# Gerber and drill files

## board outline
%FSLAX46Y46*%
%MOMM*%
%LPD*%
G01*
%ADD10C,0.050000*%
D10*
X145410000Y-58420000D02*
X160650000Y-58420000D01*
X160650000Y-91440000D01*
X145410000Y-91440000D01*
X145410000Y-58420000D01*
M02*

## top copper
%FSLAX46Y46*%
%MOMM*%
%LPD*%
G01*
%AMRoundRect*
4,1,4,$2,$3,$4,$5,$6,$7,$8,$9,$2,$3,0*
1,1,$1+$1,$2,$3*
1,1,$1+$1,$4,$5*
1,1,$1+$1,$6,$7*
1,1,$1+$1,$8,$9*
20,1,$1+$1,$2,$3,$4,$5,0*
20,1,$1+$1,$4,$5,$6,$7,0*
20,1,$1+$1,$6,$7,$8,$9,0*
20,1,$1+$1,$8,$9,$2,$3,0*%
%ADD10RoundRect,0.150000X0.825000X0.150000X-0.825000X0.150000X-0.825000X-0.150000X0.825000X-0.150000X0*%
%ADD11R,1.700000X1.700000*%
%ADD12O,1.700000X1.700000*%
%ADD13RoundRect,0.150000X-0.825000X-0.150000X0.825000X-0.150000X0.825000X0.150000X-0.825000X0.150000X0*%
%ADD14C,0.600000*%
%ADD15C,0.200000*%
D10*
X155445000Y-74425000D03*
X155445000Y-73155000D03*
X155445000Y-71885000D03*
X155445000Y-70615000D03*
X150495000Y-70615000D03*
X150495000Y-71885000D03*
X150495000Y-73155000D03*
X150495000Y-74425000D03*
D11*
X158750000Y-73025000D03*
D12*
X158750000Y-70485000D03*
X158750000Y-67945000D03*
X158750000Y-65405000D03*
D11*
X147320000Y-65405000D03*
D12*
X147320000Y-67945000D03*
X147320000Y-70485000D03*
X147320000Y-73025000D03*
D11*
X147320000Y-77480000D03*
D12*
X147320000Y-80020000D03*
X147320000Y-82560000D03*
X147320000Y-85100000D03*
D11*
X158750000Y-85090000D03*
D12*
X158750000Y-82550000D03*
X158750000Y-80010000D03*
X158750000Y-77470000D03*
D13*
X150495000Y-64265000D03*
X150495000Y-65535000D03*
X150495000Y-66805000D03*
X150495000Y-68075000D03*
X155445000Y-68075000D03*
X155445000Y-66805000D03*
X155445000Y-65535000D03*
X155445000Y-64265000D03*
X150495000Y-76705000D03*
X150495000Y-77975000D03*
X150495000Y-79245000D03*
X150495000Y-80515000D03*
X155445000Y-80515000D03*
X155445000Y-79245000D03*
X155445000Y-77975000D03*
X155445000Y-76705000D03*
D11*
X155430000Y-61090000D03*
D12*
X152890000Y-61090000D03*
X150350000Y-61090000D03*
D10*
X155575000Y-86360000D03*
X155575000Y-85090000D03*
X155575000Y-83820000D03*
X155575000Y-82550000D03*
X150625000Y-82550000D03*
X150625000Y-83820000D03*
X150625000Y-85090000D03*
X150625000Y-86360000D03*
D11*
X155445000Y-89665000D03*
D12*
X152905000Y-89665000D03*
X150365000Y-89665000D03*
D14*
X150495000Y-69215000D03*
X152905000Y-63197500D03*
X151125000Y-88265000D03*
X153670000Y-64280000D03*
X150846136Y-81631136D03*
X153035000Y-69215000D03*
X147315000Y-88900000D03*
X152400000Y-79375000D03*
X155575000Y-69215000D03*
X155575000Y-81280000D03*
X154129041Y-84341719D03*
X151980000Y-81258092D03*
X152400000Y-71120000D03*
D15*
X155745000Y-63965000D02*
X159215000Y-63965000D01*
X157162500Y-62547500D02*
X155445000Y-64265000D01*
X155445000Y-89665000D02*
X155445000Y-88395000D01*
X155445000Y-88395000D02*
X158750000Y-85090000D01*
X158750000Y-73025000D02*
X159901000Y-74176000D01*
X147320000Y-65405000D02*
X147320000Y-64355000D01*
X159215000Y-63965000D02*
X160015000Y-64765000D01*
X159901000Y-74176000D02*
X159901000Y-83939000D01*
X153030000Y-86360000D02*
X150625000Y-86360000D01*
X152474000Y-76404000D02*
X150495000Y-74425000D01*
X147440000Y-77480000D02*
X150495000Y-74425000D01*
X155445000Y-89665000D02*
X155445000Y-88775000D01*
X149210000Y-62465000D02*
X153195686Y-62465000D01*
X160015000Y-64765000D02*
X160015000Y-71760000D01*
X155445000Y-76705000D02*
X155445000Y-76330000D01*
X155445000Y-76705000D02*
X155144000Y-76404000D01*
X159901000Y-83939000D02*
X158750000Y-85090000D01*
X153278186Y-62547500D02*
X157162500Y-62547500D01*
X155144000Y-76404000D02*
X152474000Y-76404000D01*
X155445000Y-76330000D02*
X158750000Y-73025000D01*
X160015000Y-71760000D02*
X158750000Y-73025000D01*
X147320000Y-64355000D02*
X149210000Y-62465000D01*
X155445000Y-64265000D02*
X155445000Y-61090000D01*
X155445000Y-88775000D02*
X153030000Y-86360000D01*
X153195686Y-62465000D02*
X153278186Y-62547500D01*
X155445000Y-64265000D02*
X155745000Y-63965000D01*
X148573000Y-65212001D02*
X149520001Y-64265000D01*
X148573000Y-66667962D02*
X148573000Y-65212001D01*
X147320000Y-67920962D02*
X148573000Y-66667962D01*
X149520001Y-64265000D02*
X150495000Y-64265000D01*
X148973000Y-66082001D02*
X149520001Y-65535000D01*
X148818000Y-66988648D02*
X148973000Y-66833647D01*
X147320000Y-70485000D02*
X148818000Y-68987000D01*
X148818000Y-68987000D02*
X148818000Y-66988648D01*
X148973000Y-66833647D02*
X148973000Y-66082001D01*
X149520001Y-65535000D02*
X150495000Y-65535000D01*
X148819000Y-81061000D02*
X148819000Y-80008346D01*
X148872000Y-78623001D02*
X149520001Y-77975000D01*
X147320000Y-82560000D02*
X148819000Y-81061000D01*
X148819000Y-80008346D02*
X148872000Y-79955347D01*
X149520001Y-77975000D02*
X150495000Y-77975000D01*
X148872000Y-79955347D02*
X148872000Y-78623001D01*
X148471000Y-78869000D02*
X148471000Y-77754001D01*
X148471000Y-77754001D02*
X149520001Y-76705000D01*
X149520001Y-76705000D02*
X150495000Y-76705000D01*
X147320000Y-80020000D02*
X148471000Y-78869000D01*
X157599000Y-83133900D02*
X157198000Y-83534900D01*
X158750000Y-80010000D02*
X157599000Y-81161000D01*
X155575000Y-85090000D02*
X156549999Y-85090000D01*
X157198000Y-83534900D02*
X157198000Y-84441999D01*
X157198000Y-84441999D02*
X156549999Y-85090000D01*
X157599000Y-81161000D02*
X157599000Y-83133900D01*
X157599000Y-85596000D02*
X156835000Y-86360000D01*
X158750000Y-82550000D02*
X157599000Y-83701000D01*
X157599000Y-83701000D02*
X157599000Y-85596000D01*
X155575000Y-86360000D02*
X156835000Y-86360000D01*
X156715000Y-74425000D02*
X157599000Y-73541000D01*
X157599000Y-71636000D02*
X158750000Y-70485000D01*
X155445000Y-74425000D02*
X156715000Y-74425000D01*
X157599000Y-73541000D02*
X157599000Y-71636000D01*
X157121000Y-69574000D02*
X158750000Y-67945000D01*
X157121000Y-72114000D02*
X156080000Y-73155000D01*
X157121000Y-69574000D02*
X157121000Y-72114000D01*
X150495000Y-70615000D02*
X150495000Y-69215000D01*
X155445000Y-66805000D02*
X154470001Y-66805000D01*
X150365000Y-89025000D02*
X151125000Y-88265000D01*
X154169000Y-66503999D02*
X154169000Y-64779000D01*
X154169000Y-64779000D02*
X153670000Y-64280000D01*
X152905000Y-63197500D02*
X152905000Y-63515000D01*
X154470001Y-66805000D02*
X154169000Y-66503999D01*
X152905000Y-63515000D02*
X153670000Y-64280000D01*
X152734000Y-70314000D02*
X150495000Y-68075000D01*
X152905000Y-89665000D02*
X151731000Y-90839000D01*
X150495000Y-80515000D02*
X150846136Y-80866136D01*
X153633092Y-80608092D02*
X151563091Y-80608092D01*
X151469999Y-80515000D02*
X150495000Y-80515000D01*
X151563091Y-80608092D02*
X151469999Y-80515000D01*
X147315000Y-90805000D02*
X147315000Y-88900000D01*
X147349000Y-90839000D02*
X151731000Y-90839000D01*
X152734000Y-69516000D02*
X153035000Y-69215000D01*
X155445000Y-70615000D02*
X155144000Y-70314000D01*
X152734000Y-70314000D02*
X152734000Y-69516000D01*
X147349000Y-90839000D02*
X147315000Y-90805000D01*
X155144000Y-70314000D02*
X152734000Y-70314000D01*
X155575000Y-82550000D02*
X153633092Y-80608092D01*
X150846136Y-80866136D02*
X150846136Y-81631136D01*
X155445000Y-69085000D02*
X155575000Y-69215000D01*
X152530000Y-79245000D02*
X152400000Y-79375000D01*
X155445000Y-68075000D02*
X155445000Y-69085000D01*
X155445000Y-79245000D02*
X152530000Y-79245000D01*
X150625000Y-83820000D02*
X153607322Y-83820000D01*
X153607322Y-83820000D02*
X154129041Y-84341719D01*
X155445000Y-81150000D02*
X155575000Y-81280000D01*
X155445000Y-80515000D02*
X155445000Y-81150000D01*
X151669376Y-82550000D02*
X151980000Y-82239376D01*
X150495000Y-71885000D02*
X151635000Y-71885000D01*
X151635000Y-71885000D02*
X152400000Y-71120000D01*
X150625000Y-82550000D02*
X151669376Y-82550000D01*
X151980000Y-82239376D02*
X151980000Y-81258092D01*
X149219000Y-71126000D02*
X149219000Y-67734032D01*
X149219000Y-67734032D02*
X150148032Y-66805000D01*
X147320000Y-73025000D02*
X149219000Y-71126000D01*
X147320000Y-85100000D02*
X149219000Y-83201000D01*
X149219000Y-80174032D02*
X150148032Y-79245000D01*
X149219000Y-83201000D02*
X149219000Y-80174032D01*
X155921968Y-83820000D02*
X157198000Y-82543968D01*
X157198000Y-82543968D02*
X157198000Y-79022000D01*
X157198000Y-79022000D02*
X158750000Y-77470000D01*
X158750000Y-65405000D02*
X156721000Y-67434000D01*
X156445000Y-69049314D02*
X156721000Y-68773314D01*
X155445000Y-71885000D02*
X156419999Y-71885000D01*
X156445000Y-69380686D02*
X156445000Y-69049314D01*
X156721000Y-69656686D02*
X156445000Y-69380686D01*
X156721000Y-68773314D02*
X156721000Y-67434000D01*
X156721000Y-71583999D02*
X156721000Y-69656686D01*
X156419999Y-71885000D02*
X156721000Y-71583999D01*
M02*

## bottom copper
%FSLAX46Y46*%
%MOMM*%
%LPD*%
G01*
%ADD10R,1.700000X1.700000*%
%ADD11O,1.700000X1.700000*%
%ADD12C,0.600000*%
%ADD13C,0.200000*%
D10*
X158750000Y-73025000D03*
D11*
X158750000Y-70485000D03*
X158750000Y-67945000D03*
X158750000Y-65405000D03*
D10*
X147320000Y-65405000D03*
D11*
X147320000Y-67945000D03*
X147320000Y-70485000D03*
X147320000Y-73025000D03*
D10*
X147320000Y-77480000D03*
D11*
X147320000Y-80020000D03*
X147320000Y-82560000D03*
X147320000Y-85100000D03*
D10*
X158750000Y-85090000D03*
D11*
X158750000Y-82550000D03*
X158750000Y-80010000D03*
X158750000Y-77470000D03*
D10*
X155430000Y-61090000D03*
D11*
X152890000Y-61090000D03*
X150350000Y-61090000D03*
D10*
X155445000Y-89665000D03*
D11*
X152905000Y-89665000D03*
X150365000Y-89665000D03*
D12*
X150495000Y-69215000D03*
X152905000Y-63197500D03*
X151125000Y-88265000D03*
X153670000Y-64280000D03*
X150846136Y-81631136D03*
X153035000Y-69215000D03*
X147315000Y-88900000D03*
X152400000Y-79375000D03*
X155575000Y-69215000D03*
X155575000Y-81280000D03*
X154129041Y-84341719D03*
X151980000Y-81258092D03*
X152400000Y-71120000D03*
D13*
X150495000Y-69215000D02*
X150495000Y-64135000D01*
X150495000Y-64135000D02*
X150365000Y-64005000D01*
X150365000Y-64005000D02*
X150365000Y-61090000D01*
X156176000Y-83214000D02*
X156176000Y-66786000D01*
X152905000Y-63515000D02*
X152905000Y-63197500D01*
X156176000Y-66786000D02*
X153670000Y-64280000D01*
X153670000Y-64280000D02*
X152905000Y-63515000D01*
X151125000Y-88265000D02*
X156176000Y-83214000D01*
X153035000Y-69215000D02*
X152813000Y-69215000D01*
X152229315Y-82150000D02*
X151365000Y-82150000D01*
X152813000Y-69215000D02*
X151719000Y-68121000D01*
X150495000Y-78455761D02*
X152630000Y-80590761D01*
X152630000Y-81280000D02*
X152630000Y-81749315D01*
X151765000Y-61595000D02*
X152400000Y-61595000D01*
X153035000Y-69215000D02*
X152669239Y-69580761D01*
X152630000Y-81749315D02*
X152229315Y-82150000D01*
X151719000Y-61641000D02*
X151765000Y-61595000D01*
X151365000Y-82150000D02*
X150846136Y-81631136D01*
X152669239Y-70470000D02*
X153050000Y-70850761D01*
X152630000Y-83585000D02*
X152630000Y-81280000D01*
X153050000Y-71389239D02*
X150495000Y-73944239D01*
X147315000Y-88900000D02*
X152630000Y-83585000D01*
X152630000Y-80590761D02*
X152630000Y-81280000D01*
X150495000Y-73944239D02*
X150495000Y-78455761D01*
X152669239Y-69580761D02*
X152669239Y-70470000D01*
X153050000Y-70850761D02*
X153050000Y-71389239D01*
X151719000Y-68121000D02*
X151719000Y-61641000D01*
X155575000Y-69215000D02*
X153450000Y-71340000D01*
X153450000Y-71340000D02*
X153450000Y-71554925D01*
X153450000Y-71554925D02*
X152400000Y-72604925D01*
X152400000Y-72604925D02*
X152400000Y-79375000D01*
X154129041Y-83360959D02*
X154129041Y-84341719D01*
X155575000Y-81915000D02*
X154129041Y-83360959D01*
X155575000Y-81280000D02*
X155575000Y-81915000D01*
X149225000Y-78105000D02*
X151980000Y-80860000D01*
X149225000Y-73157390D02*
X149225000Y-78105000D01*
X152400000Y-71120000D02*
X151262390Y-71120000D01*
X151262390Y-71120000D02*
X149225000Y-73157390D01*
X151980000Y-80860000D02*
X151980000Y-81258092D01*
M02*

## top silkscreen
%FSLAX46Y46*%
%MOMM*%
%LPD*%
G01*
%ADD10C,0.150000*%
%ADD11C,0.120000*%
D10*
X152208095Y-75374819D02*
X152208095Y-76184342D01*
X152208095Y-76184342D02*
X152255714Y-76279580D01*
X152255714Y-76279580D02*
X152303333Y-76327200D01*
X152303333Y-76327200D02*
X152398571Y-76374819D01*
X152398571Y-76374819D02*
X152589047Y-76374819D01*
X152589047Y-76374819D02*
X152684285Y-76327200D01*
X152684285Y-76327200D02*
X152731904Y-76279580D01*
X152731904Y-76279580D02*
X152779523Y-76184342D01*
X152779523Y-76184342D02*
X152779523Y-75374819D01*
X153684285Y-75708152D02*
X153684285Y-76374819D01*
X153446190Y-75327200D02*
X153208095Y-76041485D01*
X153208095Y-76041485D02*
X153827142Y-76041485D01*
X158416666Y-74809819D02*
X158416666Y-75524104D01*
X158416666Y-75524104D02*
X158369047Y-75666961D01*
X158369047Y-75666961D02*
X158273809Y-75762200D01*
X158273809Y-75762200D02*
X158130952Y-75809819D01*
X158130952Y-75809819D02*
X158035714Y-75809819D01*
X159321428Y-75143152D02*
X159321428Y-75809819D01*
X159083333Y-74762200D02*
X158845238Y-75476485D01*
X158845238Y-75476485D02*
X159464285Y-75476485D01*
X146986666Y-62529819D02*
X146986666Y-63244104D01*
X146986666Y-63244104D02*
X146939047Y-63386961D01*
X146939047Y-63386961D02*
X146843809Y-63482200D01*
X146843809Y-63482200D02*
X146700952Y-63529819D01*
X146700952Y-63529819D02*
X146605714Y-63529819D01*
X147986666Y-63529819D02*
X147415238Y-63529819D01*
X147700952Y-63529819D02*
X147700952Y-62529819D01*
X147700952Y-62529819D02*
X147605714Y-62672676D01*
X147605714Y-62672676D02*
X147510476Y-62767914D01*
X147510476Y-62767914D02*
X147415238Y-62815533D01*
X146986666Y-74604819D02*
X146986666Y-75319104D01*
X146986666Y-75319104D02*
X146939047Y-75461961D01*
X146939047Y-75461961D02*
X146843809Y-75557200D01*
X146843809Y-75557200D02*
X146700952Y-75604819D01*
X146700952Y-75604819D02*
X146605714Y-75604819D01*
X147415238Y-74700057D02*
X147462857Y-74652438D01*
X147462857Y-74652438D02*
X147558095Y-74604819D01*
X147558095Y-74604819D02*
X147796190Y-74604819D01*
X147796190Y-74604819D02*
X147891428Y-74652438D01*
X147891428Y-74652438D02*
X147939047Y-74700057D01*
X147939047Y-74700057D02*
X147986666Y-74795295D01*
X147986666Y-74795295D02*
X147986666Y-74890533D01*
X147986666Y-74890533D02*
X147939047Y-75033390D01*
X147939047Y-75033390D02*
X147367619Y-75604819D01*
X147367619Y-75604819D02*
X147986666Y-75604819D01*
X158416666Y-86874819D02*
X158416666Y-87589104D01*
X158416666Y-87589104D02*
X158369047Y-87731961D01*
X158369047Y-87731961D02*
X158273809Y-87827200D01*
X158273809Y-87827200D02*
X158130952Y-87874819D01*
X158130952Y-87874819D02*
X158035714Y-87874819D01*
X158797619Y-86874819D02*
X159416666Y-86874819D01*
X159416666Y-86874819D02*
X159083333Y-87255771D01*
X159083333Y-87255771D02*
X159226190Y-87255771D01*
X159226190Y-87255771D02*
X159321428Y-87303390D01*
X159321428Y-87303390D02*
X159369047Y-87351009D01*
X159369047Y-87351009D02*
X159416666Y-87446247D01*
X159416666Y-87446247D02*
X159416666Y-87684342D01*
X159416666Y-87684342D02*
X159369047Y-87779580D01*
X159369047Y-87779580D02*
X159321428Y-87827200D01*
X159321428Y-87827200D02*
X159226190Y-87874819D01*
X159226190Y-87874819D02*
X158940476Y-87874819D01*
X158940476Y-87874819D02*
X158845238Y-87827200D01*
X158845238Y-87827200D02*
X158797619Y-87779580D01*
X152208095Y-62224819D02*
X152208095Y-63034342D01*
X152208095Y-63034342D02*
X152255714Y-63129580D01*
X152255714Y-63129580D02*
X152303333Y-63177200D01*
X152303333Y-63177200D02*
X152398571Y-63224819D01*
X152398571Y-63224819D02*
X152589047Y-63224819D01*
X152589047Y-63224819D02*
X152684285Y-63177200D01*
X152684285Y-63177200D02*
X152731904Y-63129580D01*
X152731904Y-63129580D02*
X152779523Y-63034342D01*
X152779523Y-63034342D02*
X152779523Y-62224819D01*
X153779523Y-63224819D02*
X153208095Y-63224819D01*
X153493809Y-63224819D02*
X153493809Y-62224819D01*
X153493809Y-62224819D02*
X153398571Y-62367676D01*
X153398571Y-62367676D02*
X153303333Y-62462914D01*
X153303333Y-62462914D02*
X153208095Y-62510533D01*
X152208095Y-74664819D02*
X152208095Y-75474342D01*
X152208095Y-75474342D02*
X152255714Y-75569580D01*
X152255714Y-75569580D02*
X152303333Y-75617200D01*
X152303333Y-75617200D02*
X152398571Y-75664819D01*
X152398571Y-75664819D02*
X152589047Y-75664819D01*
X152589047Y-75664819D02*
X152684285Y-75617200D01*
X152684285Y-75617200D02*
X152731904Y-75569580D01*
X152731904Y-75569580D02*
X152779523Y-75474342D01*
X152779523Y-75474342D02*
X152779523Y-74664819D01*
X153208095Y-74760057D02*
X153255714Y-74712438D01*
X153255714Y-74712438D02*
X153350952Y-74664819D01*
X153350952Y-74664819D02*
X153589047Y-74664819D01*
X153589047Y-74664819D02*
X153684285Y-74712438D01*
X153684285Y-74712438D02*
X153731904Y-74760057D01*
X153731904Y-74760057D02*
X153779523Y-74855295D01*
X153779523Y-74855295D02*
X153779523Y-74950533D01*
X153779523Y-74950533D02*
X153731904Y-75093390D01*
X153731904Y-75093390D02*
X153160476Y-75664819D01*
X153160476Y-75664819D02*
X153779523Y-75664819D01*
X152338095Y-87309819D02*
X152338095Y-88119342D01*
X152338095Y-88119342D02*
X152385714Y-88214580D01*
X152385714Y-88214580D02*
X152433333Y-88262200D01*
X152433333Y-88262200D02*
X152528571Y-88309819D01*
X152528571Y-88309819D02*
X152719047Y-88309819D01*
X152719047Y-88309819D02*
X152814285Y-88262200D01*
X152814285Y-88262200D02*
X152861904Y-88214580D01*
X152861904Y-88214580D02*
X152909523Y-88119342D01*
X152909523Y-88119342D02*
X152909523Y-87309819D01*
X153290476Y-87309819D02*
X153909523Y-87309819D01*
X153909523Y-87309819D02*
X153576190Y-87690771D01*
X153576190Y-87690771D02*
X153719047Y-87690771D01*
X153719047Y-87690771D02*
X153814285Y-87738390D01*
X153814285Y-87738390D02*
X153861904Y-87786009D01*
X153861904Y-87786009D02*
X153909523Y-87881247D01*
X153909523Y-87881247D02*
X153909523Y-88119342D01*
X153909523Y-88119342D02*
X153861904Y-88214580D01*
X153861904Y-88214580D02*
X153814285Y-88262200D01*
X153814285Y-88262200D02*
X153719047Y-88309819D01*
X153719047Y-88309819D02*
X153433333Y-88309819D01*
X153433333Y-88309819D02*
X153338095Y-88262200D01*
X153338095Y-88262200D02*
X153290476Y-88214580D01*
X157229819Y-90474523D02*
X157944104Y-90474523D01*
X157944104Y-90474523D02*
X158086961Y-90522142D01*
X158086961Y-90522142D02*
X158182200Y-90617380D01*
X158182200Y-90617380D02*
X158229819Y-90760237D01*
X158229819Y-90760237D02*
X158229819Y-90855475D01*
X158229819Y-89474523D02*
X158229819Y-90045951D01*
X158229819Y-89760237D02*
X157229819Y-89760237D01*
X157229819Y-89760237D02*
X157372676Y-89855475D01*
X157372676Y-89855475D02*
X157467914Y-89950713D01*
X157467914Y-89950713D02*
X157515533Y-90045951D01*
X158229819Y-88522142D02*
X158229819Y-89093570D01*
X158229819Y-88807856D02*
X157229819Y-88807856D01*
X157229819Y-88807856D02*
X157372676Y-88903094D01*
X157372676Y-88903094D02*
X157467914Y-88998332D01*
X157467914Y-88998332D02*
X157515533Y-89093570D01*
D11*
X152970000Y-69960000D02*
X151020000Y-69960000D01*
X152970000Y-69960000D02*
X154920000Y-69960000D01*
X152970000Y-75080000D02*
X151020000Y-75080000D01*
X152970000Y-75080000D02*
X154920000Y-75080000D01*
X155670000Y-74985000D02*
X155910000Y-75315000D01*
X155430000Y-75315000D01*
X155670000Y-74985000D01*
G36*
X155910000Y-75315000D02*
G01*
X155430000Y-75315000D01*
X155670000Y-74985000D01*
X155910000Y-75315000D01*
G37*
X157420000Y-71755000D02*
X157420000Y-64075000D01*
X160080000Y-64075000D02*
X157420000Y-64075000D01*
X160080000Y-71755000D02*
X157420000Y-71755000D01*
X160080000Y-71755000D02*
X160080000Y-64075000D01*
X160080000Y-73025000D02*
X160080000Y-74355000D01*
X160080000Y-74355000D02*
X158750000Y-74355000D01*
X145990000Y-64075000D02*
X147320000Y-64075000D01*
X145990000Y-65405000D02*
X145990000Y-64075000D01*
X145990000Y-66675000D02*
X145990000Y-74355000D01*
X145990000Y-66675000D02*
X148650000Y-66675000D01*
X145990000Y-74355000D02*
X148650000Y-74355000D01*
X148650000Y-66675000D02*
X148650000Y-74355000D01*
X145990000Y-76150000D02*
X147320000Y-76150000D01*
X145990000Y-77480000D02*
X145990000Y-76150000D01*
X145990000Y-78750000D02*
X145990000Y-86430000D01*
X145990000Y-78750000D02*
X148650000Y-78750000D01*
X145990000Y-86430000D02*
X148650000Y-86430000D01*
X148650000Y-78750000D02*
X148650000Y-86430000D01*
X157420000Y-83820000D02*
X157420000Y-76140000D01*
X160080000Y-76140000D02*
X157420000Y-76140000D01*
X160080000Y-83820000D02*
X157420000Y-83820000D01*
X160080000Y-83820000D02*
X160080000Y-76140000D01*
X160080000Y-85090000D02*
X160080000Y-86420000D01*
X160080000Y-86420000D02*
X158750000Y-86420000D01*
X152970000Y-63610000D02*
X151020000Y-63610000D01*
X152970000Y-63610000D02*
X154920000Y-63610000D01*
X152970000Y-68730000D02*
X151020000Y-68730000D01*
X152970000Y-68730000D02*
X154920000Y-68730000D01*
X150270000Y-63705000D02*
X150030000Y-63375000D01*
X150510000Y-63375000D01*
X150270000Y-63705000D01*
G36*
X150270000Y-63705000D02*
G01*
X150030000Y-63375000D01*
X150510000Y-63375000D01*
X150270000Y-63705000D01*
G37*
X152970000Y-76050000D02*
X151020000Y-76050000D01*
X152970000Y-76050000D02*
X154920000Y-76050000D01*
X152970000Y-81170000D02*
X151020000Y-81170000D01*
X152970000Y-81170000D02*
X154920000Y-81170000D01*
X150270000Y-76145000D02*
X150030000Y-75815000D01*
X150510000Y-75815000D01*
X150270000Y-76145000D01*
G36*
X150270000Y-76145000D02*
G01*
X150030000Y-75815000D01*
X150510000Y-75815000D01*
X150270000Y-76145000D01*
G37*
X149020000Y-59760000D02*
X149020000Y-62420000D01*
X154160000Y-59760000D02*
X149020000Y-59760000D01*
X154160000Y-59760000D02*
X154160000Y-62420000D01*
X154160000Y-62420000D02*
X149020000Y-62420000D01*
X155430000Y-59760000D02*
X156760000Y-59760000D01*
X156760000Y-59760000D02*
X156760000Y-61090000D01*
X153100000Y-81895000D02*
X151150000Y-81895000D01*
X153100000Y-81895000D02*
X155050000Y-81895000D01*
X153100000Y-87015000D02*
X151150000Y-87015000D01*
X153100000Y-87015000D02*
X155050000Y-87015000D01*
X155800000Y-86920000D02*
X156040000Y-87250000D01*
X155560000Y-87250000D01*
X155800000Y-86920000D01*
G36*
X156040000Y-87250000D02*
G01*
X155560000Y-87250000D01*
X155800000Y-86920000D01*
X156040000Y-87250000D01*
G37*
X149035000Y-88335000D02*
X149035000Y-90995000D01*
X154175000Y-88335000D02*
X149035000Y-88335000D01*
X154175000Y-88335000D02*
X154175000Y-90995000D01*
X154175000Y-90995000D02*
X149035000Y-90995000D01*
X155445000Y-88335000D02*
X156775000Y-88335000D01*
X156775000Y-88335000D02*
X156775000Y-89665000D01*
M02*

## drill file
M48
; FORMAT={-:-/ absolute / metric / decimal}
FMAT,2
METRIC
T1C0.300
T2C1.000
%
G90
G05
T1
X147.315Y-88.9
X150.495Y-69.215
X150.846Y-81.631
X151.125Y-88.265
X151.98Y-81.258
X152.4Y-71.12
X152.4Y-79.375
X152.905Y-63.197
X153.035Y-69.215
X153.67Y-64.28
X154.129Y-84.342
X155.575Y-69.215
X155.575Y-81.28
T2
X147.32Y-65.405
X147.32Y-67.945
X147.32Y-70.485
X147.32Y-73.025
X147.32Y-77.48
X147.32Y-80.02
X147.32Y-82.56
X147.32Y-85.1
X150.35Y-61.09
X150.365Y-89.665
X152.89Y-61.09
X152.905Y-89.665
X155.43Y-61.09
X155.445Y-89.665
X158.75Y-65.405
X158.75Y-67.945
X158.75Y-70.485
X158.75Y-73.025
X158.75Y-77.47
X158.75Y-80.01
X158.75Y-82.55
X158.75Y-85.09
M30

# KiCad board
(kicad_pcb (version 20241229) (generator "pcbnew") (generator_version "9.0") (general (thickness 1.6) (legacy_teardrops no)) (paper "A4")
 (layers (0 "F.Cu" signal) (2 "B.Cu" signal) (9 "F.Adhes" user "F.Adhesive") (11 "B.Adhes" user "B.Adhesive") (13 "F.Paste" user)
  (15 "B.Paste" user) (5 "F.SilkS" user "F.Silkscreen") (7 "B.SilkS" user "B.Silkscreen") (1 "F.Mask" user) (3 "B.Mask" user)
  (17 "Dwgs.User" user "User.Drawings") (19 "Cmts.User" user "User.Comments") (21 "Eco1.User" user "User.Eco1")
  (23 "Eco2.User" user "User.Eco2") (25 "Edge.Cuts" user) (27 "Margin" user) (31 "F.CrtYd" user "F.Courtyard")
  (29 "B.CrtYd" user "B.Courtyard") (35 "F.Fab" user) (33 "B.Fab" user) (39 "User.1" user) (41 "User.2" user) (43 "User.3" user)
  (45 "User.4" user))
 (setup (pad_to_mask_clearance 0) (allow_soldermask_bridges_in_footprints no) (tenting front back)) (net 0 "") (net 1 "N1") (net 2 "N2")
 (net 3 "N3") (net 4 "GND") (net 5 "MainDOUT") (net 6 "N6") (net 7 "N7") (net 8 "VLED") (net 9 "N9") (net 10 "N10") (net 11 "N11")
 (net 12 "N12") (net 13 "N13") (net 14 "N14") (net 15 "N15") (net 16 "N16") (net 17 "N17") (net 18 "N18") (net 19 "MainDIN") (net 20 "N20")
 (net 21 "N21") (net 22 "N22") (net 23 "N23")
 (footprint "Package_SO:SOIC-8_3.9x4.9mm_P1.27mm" (layer "F.Cu") (at 152.97 72.52 180)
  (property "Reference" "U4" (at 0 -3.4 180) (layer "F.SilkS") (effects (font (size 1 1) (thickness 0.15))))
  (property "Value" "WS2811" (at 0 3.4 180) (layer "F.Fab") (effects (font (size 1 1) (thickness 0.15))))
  (fp_line (start 0 2.56) (end 1.95 2.56) (stroke (width 0.12) (type solid)) (layer "F.SilkS"))
  (fp_line (start 0 2.56) (end -1.95 2.56) (stroke (width 0.12) (type solid)) (layer "F.SilkS"))
  (fp_line (start 0 -2.56) (end 1.95 -2.56) (stroke (width 0.12) (type solid)) (layer "F.SilkS"))
  (fp_line (start 0 -2.56) (end -1.95 -2.56) (stroke (width 0.12) (type solid)) (layer "F.SilkS"))
  (fp_poly
   (pts (xy -2.7 -2.465) (xy -2.94 -2.795) (xy -2.46 -2.795) (xy -2.7 -2.465)) (stroke (width 0.12) (type solid)) (fill yes)
   (layer "F.SilkS"))
  (pad "1" smd roundrect (at -2.475 -1.905 180) (size 1.95 0.6) (layers "F.Cu" "F.Mask" "F.Paste") (roundrect_rratio 0.25) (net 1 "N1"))
  (pad "2" smd roundrect (at -2.475 -0.635 180) (size 1.95 0.6) (layers "F.Cu" "F.Mask" "F.Paste") (roundrect_rratio 0.25) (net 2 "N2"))
  (pad "3" smd roundrect (at -2.475 0.635 180) (size 1.95 0.6) (layers "F.Cu" "F.Mask" "F.Paste") (roundrect_rratio 0.25) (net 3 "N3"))
  (pad "4" smd roundrect (at -2.475 1.905 180) (size 1.95 0.6) (layers "F.Cu" "F.Mask" "F.Paste") (roundrect_rratio 0.25) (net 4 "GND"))
  (pad "5" smd roundrect (at 2.475 1.905 180) (size 1.95 0.6) (layers "F.Cu" "F.Mask" "F.Paste") (roundrect_rratio 0.25) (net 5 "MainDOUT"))
  (pad "6" smd roundrect (at 2.475 0.635 180) (size 1.95 0.6) (layers "F.Cu" "F.Mask" "F.Paste") (roundrect_rratio 0.25) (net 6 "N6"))
  (pad "7" smd roundrect (at 2.475 -0.635 180) (size 1.95 0.6) (layers "F.Cu" "F.Mask" "F.Paste") (roundrect_rratio 0.25) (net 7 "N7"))
  (pad "8" smd roundrect (at 2.475 -1.905 180) (size 1.95 0.6) (layers "F.Cu" "F.Mask" "F.Paste") (roundrect_rratio 0.25) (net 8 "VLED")))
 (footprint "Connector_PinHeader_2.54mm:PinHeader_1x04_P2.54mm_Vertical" (layer "F.Cu") (at 158.75 73.025 180)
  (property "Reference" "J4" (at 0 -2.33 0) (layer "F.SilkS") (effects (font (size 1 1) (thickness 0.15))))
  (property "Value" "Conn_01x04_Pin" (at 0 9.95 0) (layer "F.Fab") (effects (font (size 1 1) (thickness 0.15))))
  (fp_line (start 1.33 1.27) (end 1.33 8.95) (stroke (width 0.12) (type solid)) (layer "F.SilkS"))
  (fp_line (start -1.33 8.95) (end 1.33 8.95) (stroke (width 0.12) (type solid)) (layer "F.SilkS"))
  (fp_line (start -1.33 1.27) (end 1.33 1.27) (stroke (width 0.12) (type solid)) (layer "F.SilkS"))
  (fp_line (start -1.33 1.27) (end -1.33 8.95) (stroke (width 0.12) (type solid)) (layer "F.SilkS"))
  (fp_line (start -1.33 0) (end -1.33 -1.33) (stroke (width 0.12) (type solid)) (layer "F.SilkS"))
  (fp_line (start -1.33 -1.33) (end 0 -1.33) (stroke (width 0.12) (type solid)) (layer "F.SilkS"))
  (pad "1" thru_hole rect (at 0 0 180) (size 1.7 1.7) (drill 1) (layers "*.Cu" "*.Mask") (remove_unused_layers no) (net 8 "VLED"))
  (pad "2" thru_hole oval (at 0 2.54 180) (size 1.7 1.7) (drill 1) (layers "*.Cu" "*.Mask") (remove_unused_layers no) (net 1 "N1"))
  (pad "3" thru_hole oval (at 0 5.08 180) (size 1.7 1.7) (drill 1) (layers "*.Cu" "*.Mask") (remove_unused_layers no) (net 2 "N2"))
  (pad "4" thru_hole oval (at 0 7.62 180) (size 1.7 1.7) (drill 1) (layers "*.Cu" "*.Mask") (remove_unused_layers no) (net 3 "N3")))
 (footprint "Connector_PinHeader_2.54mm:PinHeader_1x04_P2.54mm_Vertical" (layer "F.Cu") (at 147.32 65.405)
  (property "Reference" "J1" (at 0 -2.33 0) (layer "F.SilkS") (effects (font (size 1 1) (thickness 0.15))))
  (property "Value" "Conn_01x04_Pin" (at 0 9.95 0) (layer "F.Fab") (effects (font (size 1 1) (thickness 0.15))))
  (fp_line (start -1.33 -1.33) (end 0 -1.33) (stroke (width 0.12) (type solid)) (layer "F.SilkS"))
  (fp_line (start -1.33 0) (end -1.33 -1.33) (stroke (width 0.12) (type solid)) (layer "F.SilkS"))
  (fp_line (start -1.33 1.27) (end -1.33 8.95) (stroke (width 0.12) (type solid)) (layer "F.SilkS"))
  (fp_line (start -1.33 1.27) (end 1.33 1.27) (stroke (width 0.12) (type solid)) (layer "F.SilkS"))
  (fp_line (start -1.33 8.95) (end 1.33 8.95) (stroke (width 0.12) (type solid)) (layer "F.SilkS"))
  (fp_line (start 1.33 1.27) (end 1.33 8.95) (stroke (width 0.12) (type solid)) (layer "F.SilkS"))
  (pad "1" thru_hole rect (at 0 0) (size 1.7 1.7) (drill 1) (layers "*.Cu" "*.Mask") (remove_unused_layers no) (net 8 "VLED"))
  (pad "2" thru_hole oval (at 0 2.54) (size 1.7 1.7) (drill 1) (layers "*.Cu" "*.Mask") (remove_unused_layers no) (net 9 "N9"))
  (pad "3" thru_hole oval (at 0 5.08) (size 1.7 1.7) (drill 1) (layers "*.Cu" "*.Mask") (remove_unused_layers no) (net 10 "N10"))
  (pad "4" thru_hole oval (at 0 7.62) (size 1.7 1.7) (drill 1) (layers "*.Cu" "*.Mask") (remove_unused_layers no) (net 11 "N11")))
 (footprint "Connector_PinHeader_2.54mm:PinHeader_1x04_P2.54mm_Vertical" (layer "F.Cu") (at 147.32 77.48)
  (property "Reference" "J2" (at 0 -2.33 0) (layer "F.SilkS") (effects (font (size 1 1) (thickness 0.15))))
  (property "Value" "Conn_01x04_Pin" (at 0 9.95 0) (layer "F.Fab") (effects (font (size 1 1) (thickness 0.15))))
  (fp_line (start -1.33 -1.33) (end 0 -1.33) (stroke (width 0.12) (type solid)) (layer "F.SilkS"))
  (fp_line (start -1.33 0) (end -1.33 -1.33) (stroke (width 0.12) (type solid)) (layer "F.SilkS"))
  (fp_line (start -1.33 1.27) (end -1.33 8.95) (stroke (width 0.12) (type solid)) (layer "F.SilkS"))
  (fp_line (start -1.33 1.27) (end 1.33 1.27) (stroke (width 0.12) (type solid)) (layer "F.SilkS"))
  (fp_line (start -1.33 8.95) (end 1.33 8.95) (stroke (width 0.12) (type solid)) (layer "F.SilkS"))
  (fp_line (start 1.33 1.27) (end 1.33 8.95) (stroke (width 0.12) (type solid)) (layer "F.SilkS"))
  (pad "1" thru_hole rect (at 0 0) (size 1.7 1.7) (drill 1) (layers "*.Cu" "*.Mask") (remove_unused_layers no) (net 8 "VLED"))
  (pad "2" thru_hole oval (at 0 2.54) (size 1.7 1.7) (drill 1) (layers "*.Cu" "*.Mask") (remove_unused_layers no) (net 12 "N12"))
  (pad "3" thru_hole oval (at 0 5.08) (size 1.7 1.7) (drill 1) (layers "*.Cu" "*.Mask") (remove_unused_layers no) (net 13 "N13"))
  (pad "4" thru_hole oval (at 0 7.62) (size 1.7 1.7) (drill 1) (layers "*.Cu" "*.Mask") (remove_unused_layers no) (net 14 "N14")))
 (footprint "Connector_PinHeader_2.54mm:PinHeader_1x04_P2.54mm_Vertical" (layer "F.Cu") (at 158.75 85.09 180)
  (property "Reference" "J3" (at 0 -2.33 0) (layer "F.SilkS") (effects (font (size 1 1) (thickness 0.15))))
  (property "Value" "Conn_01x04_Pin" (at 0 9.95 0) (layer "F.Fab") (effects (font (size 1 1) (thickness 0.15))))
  (fp_line (start 1.33 1.27) (end 1.33 8.95) (stroke (width 0.12) (type solid)) (layer "F.SilkS"))
  (fp_line (start -1.33 8.95) (end 1.33 8.95) (stroke (width 0.12) (type solid)) (layer "F.SilkS"))
  (fp_line (start -1.33 1.27) (end 1.33 1.27) (stroke (width 0.12) (type solid)) (layer "F.SilkS"))
  (fp_line (start -1.33 1.27) (end -1.33 8.95) (stroke (width 0.12) (type solid)) (layer "F.SilkS"))
  (fp_line (start -1.33 0) (end -1.33 -1.33) (stroke (width 0.12) (type solid)) (layer "F.SilkS"))
  (fp_line (start -1.33 -1.33) (end 0 -1.33) (stroke (width 0.12) (type solid)) (layer "F.SilkS"))
  (pad "1" thru_hole rect (at 0 0 180) (size 1.7 1.7) (drill 1) (layers "*.Cu" "*.Mask") (remove_unused_layers no) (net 8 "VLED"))
  (pad "2" thru_hole oval (at 0 2.54 180) (size 1.7 1.7) (drill 1) (layers "*.Cu" "*.Mask") (remove_unused_layers no) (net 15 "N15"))
  (pad "3" thru_hole oval (at 0 5.08 180) (size 1.7 1.7) (drill 1) (layers "*.Cu" "*.Mask") (remove_unused_layers no) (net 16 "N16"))
  (pad "4" thru_hole oval (at 0 7.62 180) (size 1.7 1.7) (drill 1) (layers "*.Cu" "*.Mask") (remove_unused_layers no) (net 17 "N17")))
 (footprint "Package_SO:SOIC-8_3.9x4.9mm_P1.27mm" (layer "F.Cu") (at 152.97 66.17)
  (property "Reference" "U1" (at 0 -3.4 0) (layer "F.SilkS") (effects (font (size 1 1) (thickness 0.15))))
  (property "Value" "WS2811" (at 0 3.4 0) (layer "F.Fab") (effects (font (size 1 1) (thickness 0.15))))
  (fp_line (start 0 -2.56) (end -1.95 -2.56) (stroke (width 0.12) (type solid)) (layer "F.SilkS"))
  (fp_line (start 0 -2.56) (end 1.95 -2.56) (stroke (width 0.12) (type solid)) (layer "F.SilkS"))
  (fp_line (start 0 2.56) (end -1.95 2.56) (stroke (width 0.12) (type solid)) (layer "F.SilkS"))
  (fp_line (start 0 2.56) (end 1.95 2.56) (stroke (width 0.12) (type solid)) (layer "F.SilkS"))
  (fp_poly
   (pts (xy -2.7 -2.465) (xy -2.94 -2.795) (xy -2.46 -2.795) (xy -2.7 -2.465)) (stroke (width 0.12) (type solid)) (fill yes)
   (layer "F.SilkS"))
  (pad "1" smd roundrect (at -2.475 -1.905) (size 1.95 0.6) (layers "F.Cu" "F.Mask" "F.Paste") (roundrect_rratio 0.25) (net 9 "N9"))
  (pad "2" smd roundrect (at -2.475 -0.635) (size 1.95 0.6) (layers "F.Cu" "F.Mask" "F.Paste") (roundrect_rratio 0.25) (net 10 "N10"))
  (pad "3" smd roundrect (at -2.475 0.635) (size 1.95 0.6) (layers "F.Cu" "F.Mask" "F.Paste") (roundrect_rratio 0.25) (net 11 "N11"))
  (pad "4" smd roundrect (at -2.475 1.905) (size 1.95 0.6) (layers "F.Cu" "F.Mask" "F.Paste") (roundrect_rratio 0.25) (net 4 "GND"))
  (pad "5" smd roundrect (at 2.475 1.905) (size 1.95 0.6) (layers "F.Cu" "F.Mask" "F.Paste") (roundrect_rratio 0.25) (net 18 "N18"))
  (pad "6" smd roundrect (at 2.475 0.635) (size 1.95 0.6) (layers "F.Cu" "F.Mask" "F.Paste") (roundrect_rratio 0.25) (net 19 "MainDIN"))
  (pad "7" smd roundrect (at 2.475 -0.635) (size 1.95 0.6) (layers "F.Cu" "F.Mask" "F.Paste") (roundrect_rratio 0.25) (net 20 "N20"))
  (pad "8" smd roundrect (at 2.475 -1.905) (size 1.95 0.6) (layers "F.Cu" "F.Mask" "F.Paste") (roundrect_rratio 0.25) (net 8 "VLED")))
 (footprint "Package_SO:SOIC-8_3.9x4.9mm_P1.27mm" (layer "F.Cu") (at 152.97 78.61)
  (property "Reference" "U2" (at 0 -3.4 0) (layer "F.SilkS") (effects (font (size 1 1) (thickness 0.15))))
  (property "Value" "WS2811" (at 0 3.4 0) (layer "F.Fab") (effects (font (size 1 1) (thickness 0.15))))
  (fp_line (start 0 -2.56) (end -1.95 -2.56) (stroke (width 0.12) (type solid)) (layer "F.SilkS"))
  (fp_line (start 0 -2.56) (end 1.95 -2.56) (stroke (width 0.12) (type solid)) (layer "F.SilkS"))
  (fp_line (start 0 2.56) (end -1.95 2.56) (stroke (width 0.12) (type solid)) (layer "F.SilkS"))
  (fp_line (start 0 2.56) (end 1.95 2.56) (stroke (width 0.12) (type solid)) (layer "F.SilkS"))
  (fp_poly
   (pts (xy -2.7 -2.465) (xy -2.94 -2.795) (xy -2.46 -2.795) (xy -2.7 -2.465)) (stroke (width 0.12) (type solid)) (fill yes)
   (layer "F.SilkS"))
  (pad "1" smd roundrect (at -2.475 -1.905) (size 1.95 0.6) (layers "F.Cu" "F.Mask" "F.Paste") (roundrect_rratio 0.25) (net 12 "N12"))
  (pad "2" smd roundrect (at -2.475 -0.635) (size 1.95 0.6) (layers "F.Cu" "F.Mask" "F.Paste") (roundrect_rratio 0.25) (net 13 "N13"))
  (pad "3" smd roundrect (at -2.475 0.635) (size 1.95 0.6) (layers "F.Cu" "F.Mask" "F.Paste") (roundrect_rratio 0.25) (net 14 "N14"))
  (pad "4" smd roundrect (at -2.475 1.905) (size 1.95 0.6) (layers "F.Cu" "F.Mask" "F.Paste") (roundrect_rratio 0.25) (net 4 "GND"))
  (pad "5" smd roundrect (at 2.475 1.905) (size 1.95 0.6) (layers "F.Cu" "F.Mask" "F.Paste") (roundrect_rratio 0.25) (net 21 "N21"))
  (pad "6" smd roundrect (at 2.475 0.635) (size 1.95 0.6) (layers "F.Cu" "F.Mask" "F.Paste") (roundrect_rratio 0.25) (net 18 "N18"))
  (pad "7" smd roundrect (at 2.475 -0.635) (size 1.95 0.6) (layers "F.Cu" "F.Mask" "F.Paste") (roundrect_rratio 0.25) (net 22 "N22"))
  (pad "8" smd roundrect (at 2.475 -1.905) (size 1.95 0.6) (layers "F.Cu" "F.Mask" "F.Paste") (roundrect_rratio 0.25) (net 8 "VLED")))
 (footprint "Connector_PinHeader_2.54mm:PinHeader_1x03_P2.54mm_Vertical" (layer "F.Cu") (at 155.43 61.09 -90)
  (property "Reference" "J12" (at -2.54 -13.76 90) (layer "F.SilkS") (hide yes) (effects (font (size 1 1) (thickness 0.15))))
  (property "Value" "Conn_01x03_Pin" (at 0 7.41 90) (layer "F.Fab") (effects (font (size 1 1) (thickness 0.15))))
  (fp_line (start -1.33 6.41) (end 1.33 6.41) (stroke (width 0.12) (type solid)) (layer "F.SilkS"))
  (fp_line (start -1.33 1.27) (end -1.33 6.41) (stroke (width 0.12) (type solid)) (layer "F.SilkS"))
  (fp_line (start -1.33 1.27) (end 1.33 1.27) (stroke (width 0.12) (type solid)) (layer "F.SilkS"))
  (fp_line (start 1.33 1.27) (end 1.33 6.41) (stroke (width 0.12) (type solid)) (layer "F.SilkS"))
  (fp_line (start -1.33 0) (end -1.33 -1.33) (stroke (width 0.12) (type solid)) (layer "F.SilkS"))
  (fp_line (start -1.33 -1.33) (end 0 -1.33) (stroke (width 0.12) (type solid)) (layer "F.SilkS"))
  (pad "1" thru_hole rect (at 0 0 270) (size 1.7 1.7) (drill 1) (layers "*.Cu" "*.Mask") (remove_unused_layers no) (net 8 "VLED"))
  (pad "2" thru_hole oval (at 0 2.54 270) (size 1.7 1.7) (drill 1) (layers "*.Cu" "*.Mask") (remove_unused_layers no) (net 4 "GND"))
  (pad "3" thru_hole oval (at 0 5.08 270) (size 1.7 1.7) (drill 1) (layers "*.Cu" "*.Mask") (remove_unused_layers no) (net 5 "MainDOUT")))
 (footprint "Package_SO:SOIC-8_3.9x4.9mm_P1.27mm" (layer "F.Cu") (at 153.1 84.455 180)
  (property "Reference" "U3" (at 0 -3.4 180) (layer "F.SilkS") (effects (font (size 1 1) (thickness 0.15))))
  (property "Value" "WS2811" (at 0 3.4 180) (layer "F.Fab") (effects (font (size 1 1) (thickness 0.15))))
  (fp_line (start 0 2.56) (end 1.95 2.56) (stroke (width 0.12) (type solid)) (layer "F.SilkS"))
  (fp_line (start 0 2.56) (end -1.95 2.56) (stroke (width 0.12) (type solid)) (layer "F.SilkS"))
  (fp_line (start 0 -2.56) (end 1.95 -2.56) (stroke (width 0.12) (type solid)) (layer "F.SilkS"))
  (fp_line (start 0 -2.56) (end -1.95 -2.56) (stroke (width 0.12) (type solid)) (layer "F.SilkS"))
  (fp_poly
   (pts (xy -2.7 -2.465) (xy -2.94 -2.795) (xy -2.46 -2.795) (xy -2.7 -2.465)) (stroke (width 0.12) (type solid)) (fill yes)
   (layer "F.SilkS"))
  (pad "1" smd roundrect (at -2.475 -1.905 180) (size 1.95 0.6) (layers "F.Cu" "F.Mask" "F.Paste") (roundrect_rratio 0.25) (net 15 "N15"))
  (pad "2" smd roundrect (at -2.475 -0.635 180) (size 1.95 0.6) (layers "F.Cu" "F.Mask" "F.Paste") (roundrect_rratio 0.25) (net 16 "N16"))
  (pad "3" smd roundrect (at -2.475 0.635 180) (size 1.95 0.6) (layers "F.Cu" "F.Mask" "F.Paste") (roundrect_rratio 0.25) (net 17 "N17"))
  (pad "4" smd roundrect (at -2.475 1.905 180) (size 1.95 0.6) (layers "F.Cu" "F.Mask" "F.Paste") (roundrect_rratio 0.25) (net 4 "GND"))
  (pad "5" smd roundrect (at 2.475 1.905 180) (size 1.95 0.6) (layers "F.Cu" "F.Mask" "F.Paste") (roundrect_rratio 0.25) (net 6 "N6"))
  (pad "6" smd roundrect (at 2.475 0.635 180) (size 1.95 0.6) (layers "F.Cu" "F.Mask" "F.Paste") (roundrect_rratio 0.25) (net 21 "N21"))
  (pad "7" smd roundrect (at 2.475 -0.635 180) (size 1.95 0.6) (layers "F.Cu" "F.Mask" "F.Paste") (roundrect_rratio 0.25) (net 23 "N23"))
  (pad "8" smd roundrect (at 2.475 -1.905 180) (size 1.95 0.6) (layers "F.Cu" "F.Mask" "F.Paste") (roundrect_rratio 0.25) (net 8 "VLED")))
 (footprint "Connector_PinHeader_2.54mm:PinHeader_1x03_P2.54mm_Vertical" (layer "F.Cu") (at 155.445 89.665 -90)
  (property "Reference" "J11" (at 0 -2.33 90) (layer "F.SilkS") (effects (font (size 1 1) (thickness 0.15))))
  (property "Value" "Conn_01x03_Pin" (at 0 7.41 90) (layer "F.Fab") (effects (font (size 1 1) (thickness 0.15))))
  (fp_line (start -1.33 6.41) (end 1.33 6.41) (stroke (width 0.12) (type solid)) (layer "F.SilkS"))
  (fp_line (start -1.33 1.27) (end -1.33 6.41) (stroke (width 0.12) (type solid)) (layer "F.SilkS"))
  (fp_line (start -1.33 1.27) (end 1.33 1.27) (stroke (width 0.12) (type solid)) (layer "F.SilkS"))
  (fp_line (start 1.33 1.27) (end 1.33 6.41) (stroke (width 0.12) (type solid)) (layer "F.SilkS"))
  (fp_line (start -1.33 0) (end -1.33 -1.33) (stroke (width 0.12) (type solid)) (layer "F.SilkS"))
  (fp_line (start -1.33 -1.33) (end 0 -1.33) (stroke (width 0.12) (type solid)) (layer "F.SilkS"))
  (pad "1" thru_hole rect (at 0 0 270) (size 1.7 1.7) (drill 1) (layers "*.Cu" "*.Mask") (remove_unused_layers no) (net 8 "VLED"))
  (pad "2" thru_hole oval (at 0 2.54 270) (size 1.7 1.7) (drill 1) (layers "*.Cu" "*.Mask") (remove_unused_layers no) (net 4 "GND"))
  (pad "3" thru_hole oval (at 0 5.08 270) (size 1.7 1.7) (drill 1) (layers "*.Cu" "*.Mask") (remove_unused_layers no) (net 19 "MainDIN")))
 (gr_rect (start 145.41 58.42) (end 160.65 91.44) (stroke (width 0.05) (type default)) (fill no) (layer "Edge.Cuts"))
 (segment (start 155.745 63.965) (end 159.215 63.965) (width 0.2) (layer "F.Cu") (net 8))
 (segment (start 157.1625 62.5475) (end 155.445 64.265) (width 0.2) (layer "F.Cu") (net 8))
 (segment (start 155.445 89.665) (end 155.445 88.395) (width 0.2) (layer "F.Cu") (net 8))
 (segment (start 155.445 88.395) (end 158.75 85.09) (width 0.2) (layer "F.Cu") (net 8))
 (segment (start 158.75 73.025) (end 159.901 74.176) (width 0.2) (layer "F.Cu") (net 8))
 (segment (start 147.32 65.405) (end 147.32 64.355) (width 0.2) (layer "F.Cu") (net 8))
 (segment (start 159.215 63.965) (end 160.015 64.765) (width 0.2) (layer "F.Cu") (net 8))
 (segment (start 159.901 74.176) (end 159.901 83.939) (width 0.2) (layer "F.Cu") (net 8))
 (segment (start 153.03 86.36) (end 150.625 86.36) (width 0.2) (layer "F.Cu") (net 8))
 (segment (start 152.474 76.404) (end 150.495 74.425) (width 0.2) (layer "F.Cu") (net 8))
 (segment (start 147.44 77.48) (end 150.495 74.425) (width 0.2) (layer "F.Cu") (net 8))
 (segment (start 155.445 89.665) (end 155.445 88.775) (width 0.2) (layer "F.Cu") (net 8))
 (segment (start 149.21 62.465) (end 153.195686 62.465) (width 0.2) (layer "F.Cu") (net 8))
 (segment (start 160.015 64.765) (end 160.015 71.76) (width 0.2) (layer "F.Cu") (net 8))
 (segment (start 155.445 76.705) (end 155.445 76.33) (width 0.2) (layer "F.Cu") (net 8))
 (segment (start 155.445 76.705) (end 155.144 76.404) (width 0.2) (layer "F.Cu") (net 8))
 (segment (start 159.901 83.939) (end 158.75 85.09) (width 0.2) (layer "F.Cu") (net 8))
 (segment (start 153.278186 62.5475) (end 157.1625 62.5475) (width 0.2) (layer "F.Cu") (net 8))
 (segment (start 155.144 76.404) (end 152.474 76.404) (width 0.2) (layer "F.Cu") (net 8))
 (segment (start 155.445 76.33) (end 158.75 73.025) (width 0.2) (layer "F.Cu") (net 8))
 (segment (start 160.015 71.76) (end 158.75 73.025) (width 0.2) (layer "F.Cu") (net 8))
 (segment (start 147.32 64.355) (end 149.21 62.465) (width 0.2) (layer "F.Cu") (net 8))
 (segment (start 155.445 64.265) (end 155.445 61.09) (width 0.2) (layer "F.Cu") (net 8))
 (segment (start 155.445 88.775) (end 153.03 86.36) (width 0.2) (layer "F.Cu") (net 8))
 (segment (start 153.195686 62.465) (end 153.278186 62.5475) (width 0.2) (layer "F.Cu") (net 8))
 (segment (start 155.445 64.265) (end 155.745 63.965) (width 0.2) (layer "F.Cu") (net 8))
 (segment (start 148.573 65.212001) (end 149.520001 64.265) (width 0.2) (layer "F.Cu") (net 9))
 (segment (start 148.573 66.667962) (end 148.573 65.212001) (width 0.2) (layer "F.Cu") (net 9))
 (segment (start 147.32 67.920962) (end 148.573 66.667962) (width 0.2) (layer "F.Cu") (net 9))
 (segment (start 149.520001 64.265) (end 150.495 64.265) (width 0.2) (layer "F.Cu") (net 9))
 (segment (start 148.973 66.082001) (end 149.520001 65.535) (width 0.2) (layer "F.Cu") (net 10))
 (segment (start 148.818 66.988648) (end 148.973 66.833647) (width 0.2) (layer "F.Cu") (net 10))
 (segment (start 147.32 70.485) (end 148.818 68.987) (width 0.2) (layer "F.Cu") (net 10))
 (segment (start 148.818 68.987) (end 148.818 66.988648) (width 0.2) (layer "F.Cu") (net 10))
 (segment (start 148.973 66.833647) (end 148.973 66.082001) (width 0.2) (layer "F.Cu") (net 10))
 (segment (start 149.520001 65.535) (end 150.495 65.535) (width 0.2) (layer "F.Cu") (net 10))
 (segment (start 148.819 81.061) (end 148.819 80.008346) (width 0.2) (layer "F.Cu") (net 13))
 (segment (start 148.872 78.623001) (end 149.520001 77.975) (width 0.2) (layer "F.Cu") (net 13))
 (segment (start 147.32 82.56) (end 148.819 81.061) (width 0.2) (layer "F.Cu") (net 13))
 (segment (start 148.819 80.008346) (end 148.872 79.955347) (width 0.2) (layer "F.Cu") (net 13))
 (segment (start 149.520001 77.975) (end 150.495 77.975) (width 0.2) (layer "F.Cu") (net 13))
 (segment (start 148.872 79.955347) (end 148.872 78.623001) (width 0.2) (layer "F.Cu") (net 13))
 (segment (start 148.471 78.869) (end 148.471 77.754001) (width 0.2) (layer "F.Cu") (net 12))
 (segment (start 148.471 77.754001) (end 149.520001 76.705) (width 0.2) (layer "F.Cu") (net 12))
 (segment (start 149.520001 76.705) (end 150.495 76.705) (width 0.2) (layer "F.Cu") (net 12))
 (segment (start 147.32 80.02) (end 148.471 78.869) (width 0.2) (layer "F.Cu") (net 12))
 (segment (start 157.599 83.1339) (end 157.198 83.5349) (width 0.2) (layer "F.Cu") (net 16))
 (segment (start 158.75 80.01) (end 157.599 81.161) (width 0.2) (layer "F.Cu") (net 16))
 (segment (start 155.575 85.09) (end 156.549999 85.09) (width 0.2) (layer "F.Cu") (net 16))
 (segment (start 157.198 83.5349) (end 157.198 84.441999) (width 0.2) (layer "F.Cu") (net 16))
 (segment (start 157.198 84.441999) (end 156.549999 85.09) (width 0.2) (layer "F.Cu") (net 16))
 (segment (start 157.599 81.161) (end 157.599 83.1339) (width 0.2) (layer "F.Cu") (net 16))
 (segment (start 157.599 85.596) (end 156.835 86.36) (width 0.2) (layer "F.Cu") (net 15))
 (segment (start 158.75 82.55) (end 157.599 83.701) (width 0.2) (layer "F.Cu") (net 15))
 (segment (start 157.599 83.701) (end 157.599 85.596) (width 0.2) (layer "F.Cu") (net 15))
 (segment (start 155.575 86.36) (end 156.835 86.36) (width 0.2) (layer "F.Cu") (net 15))
 (segment (start 156.715 74.425) (end 157.599 73.541) (width 0.2) (layer "F.Cu") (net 1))
 (segment (start 157.599 71.636) (end 158.75 70.485) (width 0.2) (layer "F.Cu") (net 1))
 (segment (start 155.445 74.425) (end 156.715 74.425) (width 0.2) (layer "F.Cu") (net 1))
 (segment (start 157.599 73.541) (end 157.599 71.636) (width 0.2) (layer "F.Cu") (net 1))
 (segment (start 157.121 69.574) (end 158.75 67.945) (width 0.2) (layer "F.Cu") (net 2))
 (segment (start 157.121 72.114) (end 156.08 73.155) (width 0.2) (layer "F.Cu") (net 2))
 (segment (start 157.121 69.574) (end 157.121 72.114) (width 0.2) (layer "F.Cu") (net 2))
 (segment (start 150.495 70.615) (end 150.495 69.215) (width 0.2) (layer "F.Cu") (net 5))
 (via (at 150.495 69.215) (size 0.6) (drill 0.3) (layers "F.Cu" "B.Cu") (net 5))
 (segment (start 150.495 69.215) (end 150.495 64.135) (width 0.2) (layer "B.Cu") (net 5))
 (segment (start 150.495 64.135) (end 150.365 64.005) (width 0.2) (layer "B.Cu") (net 5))
 (segment (start 150.365 64.005) (end 150.365 61.09) (width 0.2) (layer "B.Cu") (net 5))
 (segment (start 155.445 66.805) (end 154.470001 66.805) (width 0.2) (layer "F.Cu") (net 19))
 (segment (start 150.365 89.025) (end 151.125 88.265) (width 0.2) (layer "F.Cu") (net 19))
 (segment (start 154.169 66.503999) (end 154.169 64.779) (width 0.2) (layer "F.Cu") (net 19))
 (segment (start 154.169 64.779) (end 153.67 64.28) (width 0.2) (layer "F.Cu") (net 19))
 (segment (start 152.905 63.1975) (end 152.905 63.515) (width 0.2) (layer "F.Cu") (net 19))
 (segment (start 154.470001 66.805) (end 154.169 66.503999) (width 0.2) (layer "F.Cu") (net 19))
 (segment (start 152.905 63.515) (end 153.67 64.28) (width 0.2) (layer "F.Cu") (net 19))
 (via (at 152.905 63.1975) (size 0.6) (drill 0.3) (layers "F.Cu" "B.Cu") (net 19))
 (via (at 151.125 88.265) (size 0.6) (drill 0.3) (layers "F.Cu" "B.Cu") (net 19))
 (via (at 153.67 64.28) (size 0.6) (drill 0.3) (layers "F.Cu" "B.Cu") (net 19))
 (segment (start 156.176 83.214) (end 156.176 66.786) (width 0.2) (layer "B.Cu") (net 19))
 (segment (start 152.905 63.515) (end 152.905 63.1975) (width 0.2) (layer "B.Cu") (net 19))
 (segment (start 156.176 66.786) (end 153.67 64.28) (width 0.2) (layer "B.Cu") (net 19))
 (segment (start 153.67 64.28) (end 152.905 63.515) (width 0.2) (layer "B.Cu") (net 19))
 (segment (start 151.125 88.265) (end 156.176 83.214) (width 0.2) (layer "B.Cu") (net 19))
 (segment (start 152.734 70.314) (end 150.495 68.075) (width 0.2) (layer "F.Cu") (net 4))
 (segment (start 152.905 89.665) (end 151.731 90.839) (width 0.2) (layer "F.Cu") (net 4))
 (segment (start 150.495 80.515) (end 150.846136 80.866136) (width 0.2) (layer "F.Cu") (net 4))
 (segment (start 153.633092 80.608092) (end 151.563091 80.608092) (width 0.2) (layer "F.Cu") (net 4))
 (segment (start 151.469999 80.515) (end 150.495 80.515) (width 0.2) (layer "F.Cu") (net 4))
 (segment (start 151.563091 80.608092) (end 151.469999 80.515) (width 0.2) (layer "F.Cu") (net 4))
 (segment (start 147.315 90.805) (end 147.315 88.9) (width 0.2) (layer "F.Cu") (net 4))
 (segment (start 147.349 90.839) (end 151.731 90.839) (width 0.2) (layer "F.Cu") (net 4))
 (segment (start 152.734 69.516) (end 153.035 69.215) (width 0.2) (layer "F.Cu") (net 4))
 (segment (start 155.445 70.615) (end 155.144 70.314) (width 0.2) (layer "F.Cu") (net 4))
 (segment (start 152.734 70.314) (end 152.734 69.516) (width 0.2) (layer "F.Cu") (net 4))
 (segment (start 147.349 90.839) (end 147.315 90.805) (width 0.2) (layer "F.Cu") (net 4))
 (segment (start 155.144 70.314) (end 152.734 70.314) (width 0.2) (layer "F.Cu") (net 4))
 (segment (start 155.575 82.55) (end 153.633092 80.608092) (width 0.2) (layer "F.Cu") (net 4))
 (segment (start 150.846136 80.866136) (end 150.846136 81.631136) (width 0.2) (layer "F.Cu") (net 4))
 (via (at 150.846136 81.631136) (size 0.6) (drill 0.3) (layers "F.Cu" "B.Cu") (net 4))
 (via (at 153.035 69.215) (size 0.6) (drill 0.3) (layers "F.Cu" "B.Cu") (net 4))
 (via (at 147.315 88.9) (size 0.6) (drill 0.3) (layers "F.Cu" "B.Cu") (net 4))
 (segment (start 153.035 69.215) (end 152.813 69.215) (width 0.2) (layer "B.Cu") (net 4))
 (segment (start 152.229315 82.15) (end 151.365 82.15) (width 0.2) (layer "B.Cu") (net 4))
 (segment (start 152.813 69.215) (end 151.719 68.121) (width 0.2) (layer "B.Cu") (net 4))
 (segment (start 150.495 78.455761) (end 152.63 80.590761) (width 0.2) (layer "B.Cu") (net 4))
 (segment (start 152.63 81.28) (end 152.63 81.749315) (width 0.2) (layer "B.Cu") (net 4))
 (segment (start 151.765 61.595) (end 152.4 61.595) (width 0.2) (layer "B.Cu") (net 4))
 (segment (start 153.035 69.215) (end 152.669239 69.580761) (width 0.2) (layer "B.Cu") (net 4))
 (segment (start 152.63 81.749315) (end 152.229315 82.15) (width 0.2) (layer "B.Cu") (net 4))
 (segment (start 151.719 61.641) (end 151.765 61.595) (width 0.2) (layer "B.Cu") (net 4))
 (segment (start 151.365 82.15) (end 150.846136 81.631136) (width 0.2) (layer "B.Cu") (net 4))
 (segment (start 152.669239 70.47) (end 153.05 70.850761) (width 0.2) (layer "B.Cu") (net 4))
 (segment (start 152.63 83.585) (end 152.63 81.28) (width 0.2) (layer "B.Cu") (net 4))
 (segment (start 153.05 71.389239) (end 150.495 73.944239) (width 0.2) (layer "B.Cu") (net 4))
 (segment (start 147.315 88.9) (end 152.63 83.585) (width 0.2) (layer "B.Cu") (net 4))
 (segment (start 152.63 80.590761) (end 152.63 81.28) (width 0.2) (layer "B.Cu") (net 4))
 (segment (start 150.495 73.944239) (end 150.495 78.455761) (width 0.2) (layer "B.Cu") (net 4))
 (segment (start 152.669239 69.580761) (end 152.669239 70.47) (width 0.2) (layer "B.Cu") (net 4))
 (segment (start 153.05 70.850761) (end 153.05 71.389239) (width 0.2) (layer "B.Cu") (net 4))
 (segment (start 151.719 68.121) (end 151.719 61.641) (width 0.2) (layer "B.Cu") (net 4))
 (segment (start 155.445 69.085) (end 155.575 69.215) (width 0.2) (layer "F.Cu") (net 18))
 (segment (start 152.53 79.245) (end 152.4 79.375) (width 0.2) (layer "F.Cu") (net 18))
 (segment (start 155.445 68.075) (end 155.445 69.085) (width 0.2) (layer "F.Cu") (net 18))
 (segment (start 155.445 79.245) (end 152.53 79.245) (width 0.2) (layer "F.Cu") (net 18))
 (via (at 152.4 79.375) (size 0.6) (drill 0.3) (layers "F.Cu" "B.Cu") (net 18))
 (via (at 155.575 69.215) (size 0.6) (drill 0.3) (layers "F.Cu" "B.Cu") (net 18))
 (segment (start 155.575 69.215) (end 153.45 71.34) (width 0.2) (layer "B.Cu") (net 18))
 (segment (start 153.45 71.34) (end 153.45 71.554925) (width 0.2) (layer "B.Cu") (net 18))
 (segment (start 153.45 71.554925) (end 152.4 72.604925) (width 0.2) (layer "B.Cu") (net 18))
 (segment (start 152.4 72.604925) (end 152.4 79.375) (width 0.2) (layer "B.Cu") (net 18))
 (segment (start 150.625 83.82) (end 153.607322 83.82) (width 0.2) (layer "F.Cu") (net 21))
 (segment (start 153.607322 83.82) (end 154.129041 84.341719) (width 0.2) (layer "F.Cu") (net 21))
 (segment (start 155.445 81.15) (end 155.575 81.28) (width 0.2) (layer "F.Cu") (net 21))
 (segment (start 155.445 80.515) (end 155.445 81.15) (width 0.2) (layer "F.Cu") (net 21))
 (via (at 155.575 81.28) (size 0.6) (drill 0.3) (layers "F.Cu" "B.Cu") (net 21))
 (via (at 154.129041 84.341719) (size 0.6) (drill 0.3) (layers "F.Cu" "B.Cu") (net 21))
 (segment (start 154.129041 83.360959) (end 154.129041 84.341719) (width 0.2) (layer "B.Cu") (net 21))
 (segment (start 155.575 81.915) (end 154.129041 83.360959) (width 0.2) (layer "B.Cu") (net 21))
 (segment (start 155.575 81.28) (end 155.575 81.915) (width 0.2) (layer "B.Cu") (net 21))
 (segment (start 151.669376 82.55) (end 151.98 82.239376) (width 0.2) (layer "F.Cu") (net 6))
 (segment (start 150.495 71.885) (end 151.635 71.885) (width 0.2) (layer "F.Cu") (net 6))
 (segment (start 151.635 71.885) (end 152.4 71.12) (width 0.2) (layer "F.Cu") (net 6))
 (segment (start 150.625 82.55) (end 151.669376 82.55) (width 0.2) (layer "F.Cu") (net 6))
 (segment (start 151.98 82.239376) (end 151.98 81.258092) (width 0.2) (layer "F.Cu") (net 6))
 (via (at 151.98 81.258092) (size 0.6) (drill 0.3) (layers "F.Cu" "B.Cu") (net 6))
 (via (at 152.4 71.12) (size 0.6) (drill 0.3) (layers "F.Cu" "B.Cu") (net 6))
 (segment (start 149.225 78.105) (end 151.98 80.86) (width 0.2) (layer "B.Cu") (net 6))
 (segment (start 149.225 73.15739) (end 149.225 78.105) (width 0.2) (layer "B.Cu") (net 6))
 (segment (start 152.4 71.12) (end 151.26239 71.12) (width 0.2) (layer "B.Cu") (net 6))
 (segment (start 151.26239 71.12) (end 149.225 73.15739) (width 0.2) (layer "B.Cu") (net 6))
 (segment (start 151.98 80.86) (end 151.98 81.258092) (width 0.2) (layer "B.Cu") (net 6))
 (segment (start 149.219 71.126) (end 149.219 67.734032) (width 0.2) (layer "F.Cu") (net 11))
 (segment (start 149.219 67.734032) (end 150.148032 66.805) (width 0.2) (layer "F.Cu") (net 11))
 (segment (start 147.32 73.025) (end 149.219 71.126) (width 0.2) (layer "F.Cu") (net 11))
 (segment (start 147.32 85.1) (end 149.219 83.201) (width 0.2) (layer "F.Cu") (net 14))
 (segment (start 149.219 80.174032) (end 150.148032 79.245) (width 0.2) (layer "F.Cu") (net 14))
 (segment (start 149.219 83.201) (end 149.219 80.174032) (width 0.2) (layer "F.Cu") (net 14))
 (segment (start 155.921968 83.82) (end 157.198 82.543968) (width 0.2) (layer "F.Cu") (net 17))
 (segment (start 157.198 82.543968) (end 157.198 79.022) (width 0.2) (layer "F.Cu") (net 17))
 (segment (start 157.198 79.022) (end 158.75 77.47) (width 0.2) (layer "F.Cu") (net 17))
 (segment (start 158.75 65.405) (end 156.721 67.434) (width 0.2) (layer "F.Cu") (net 3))
 (segment (start 156.445 69.049314) (end 156.721 68.773314) (width 0.2) (layer "F.Cu") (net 3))
 (segment (start 155.445 71.885) (end 156.419999 71.885) (width 0.2) (layer "F.Cu") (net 3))
 (segment (start 156.445 69.380686) (end 156.445 69.049314) (width 0.2) (layer "F.Cu") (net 3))
 (segment (start 156.721 69.656686) (end 156.445 69.380686) (width 0.2) (layer "F.Cu") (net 3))
 (segment (start 156.721 68.773314) (end 156.721 67.434) (width 0.2) (layer "F.Cu") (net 3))
 (segment (start 156.721 71.583999) (end 156.721 69.656686) (width 0.2) (layer "F.Cu") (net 3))
 (segment (start 156.419999 71.885) (end 156.721 71.583999) (width 0.2) (layer "F.Cu") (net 3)))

